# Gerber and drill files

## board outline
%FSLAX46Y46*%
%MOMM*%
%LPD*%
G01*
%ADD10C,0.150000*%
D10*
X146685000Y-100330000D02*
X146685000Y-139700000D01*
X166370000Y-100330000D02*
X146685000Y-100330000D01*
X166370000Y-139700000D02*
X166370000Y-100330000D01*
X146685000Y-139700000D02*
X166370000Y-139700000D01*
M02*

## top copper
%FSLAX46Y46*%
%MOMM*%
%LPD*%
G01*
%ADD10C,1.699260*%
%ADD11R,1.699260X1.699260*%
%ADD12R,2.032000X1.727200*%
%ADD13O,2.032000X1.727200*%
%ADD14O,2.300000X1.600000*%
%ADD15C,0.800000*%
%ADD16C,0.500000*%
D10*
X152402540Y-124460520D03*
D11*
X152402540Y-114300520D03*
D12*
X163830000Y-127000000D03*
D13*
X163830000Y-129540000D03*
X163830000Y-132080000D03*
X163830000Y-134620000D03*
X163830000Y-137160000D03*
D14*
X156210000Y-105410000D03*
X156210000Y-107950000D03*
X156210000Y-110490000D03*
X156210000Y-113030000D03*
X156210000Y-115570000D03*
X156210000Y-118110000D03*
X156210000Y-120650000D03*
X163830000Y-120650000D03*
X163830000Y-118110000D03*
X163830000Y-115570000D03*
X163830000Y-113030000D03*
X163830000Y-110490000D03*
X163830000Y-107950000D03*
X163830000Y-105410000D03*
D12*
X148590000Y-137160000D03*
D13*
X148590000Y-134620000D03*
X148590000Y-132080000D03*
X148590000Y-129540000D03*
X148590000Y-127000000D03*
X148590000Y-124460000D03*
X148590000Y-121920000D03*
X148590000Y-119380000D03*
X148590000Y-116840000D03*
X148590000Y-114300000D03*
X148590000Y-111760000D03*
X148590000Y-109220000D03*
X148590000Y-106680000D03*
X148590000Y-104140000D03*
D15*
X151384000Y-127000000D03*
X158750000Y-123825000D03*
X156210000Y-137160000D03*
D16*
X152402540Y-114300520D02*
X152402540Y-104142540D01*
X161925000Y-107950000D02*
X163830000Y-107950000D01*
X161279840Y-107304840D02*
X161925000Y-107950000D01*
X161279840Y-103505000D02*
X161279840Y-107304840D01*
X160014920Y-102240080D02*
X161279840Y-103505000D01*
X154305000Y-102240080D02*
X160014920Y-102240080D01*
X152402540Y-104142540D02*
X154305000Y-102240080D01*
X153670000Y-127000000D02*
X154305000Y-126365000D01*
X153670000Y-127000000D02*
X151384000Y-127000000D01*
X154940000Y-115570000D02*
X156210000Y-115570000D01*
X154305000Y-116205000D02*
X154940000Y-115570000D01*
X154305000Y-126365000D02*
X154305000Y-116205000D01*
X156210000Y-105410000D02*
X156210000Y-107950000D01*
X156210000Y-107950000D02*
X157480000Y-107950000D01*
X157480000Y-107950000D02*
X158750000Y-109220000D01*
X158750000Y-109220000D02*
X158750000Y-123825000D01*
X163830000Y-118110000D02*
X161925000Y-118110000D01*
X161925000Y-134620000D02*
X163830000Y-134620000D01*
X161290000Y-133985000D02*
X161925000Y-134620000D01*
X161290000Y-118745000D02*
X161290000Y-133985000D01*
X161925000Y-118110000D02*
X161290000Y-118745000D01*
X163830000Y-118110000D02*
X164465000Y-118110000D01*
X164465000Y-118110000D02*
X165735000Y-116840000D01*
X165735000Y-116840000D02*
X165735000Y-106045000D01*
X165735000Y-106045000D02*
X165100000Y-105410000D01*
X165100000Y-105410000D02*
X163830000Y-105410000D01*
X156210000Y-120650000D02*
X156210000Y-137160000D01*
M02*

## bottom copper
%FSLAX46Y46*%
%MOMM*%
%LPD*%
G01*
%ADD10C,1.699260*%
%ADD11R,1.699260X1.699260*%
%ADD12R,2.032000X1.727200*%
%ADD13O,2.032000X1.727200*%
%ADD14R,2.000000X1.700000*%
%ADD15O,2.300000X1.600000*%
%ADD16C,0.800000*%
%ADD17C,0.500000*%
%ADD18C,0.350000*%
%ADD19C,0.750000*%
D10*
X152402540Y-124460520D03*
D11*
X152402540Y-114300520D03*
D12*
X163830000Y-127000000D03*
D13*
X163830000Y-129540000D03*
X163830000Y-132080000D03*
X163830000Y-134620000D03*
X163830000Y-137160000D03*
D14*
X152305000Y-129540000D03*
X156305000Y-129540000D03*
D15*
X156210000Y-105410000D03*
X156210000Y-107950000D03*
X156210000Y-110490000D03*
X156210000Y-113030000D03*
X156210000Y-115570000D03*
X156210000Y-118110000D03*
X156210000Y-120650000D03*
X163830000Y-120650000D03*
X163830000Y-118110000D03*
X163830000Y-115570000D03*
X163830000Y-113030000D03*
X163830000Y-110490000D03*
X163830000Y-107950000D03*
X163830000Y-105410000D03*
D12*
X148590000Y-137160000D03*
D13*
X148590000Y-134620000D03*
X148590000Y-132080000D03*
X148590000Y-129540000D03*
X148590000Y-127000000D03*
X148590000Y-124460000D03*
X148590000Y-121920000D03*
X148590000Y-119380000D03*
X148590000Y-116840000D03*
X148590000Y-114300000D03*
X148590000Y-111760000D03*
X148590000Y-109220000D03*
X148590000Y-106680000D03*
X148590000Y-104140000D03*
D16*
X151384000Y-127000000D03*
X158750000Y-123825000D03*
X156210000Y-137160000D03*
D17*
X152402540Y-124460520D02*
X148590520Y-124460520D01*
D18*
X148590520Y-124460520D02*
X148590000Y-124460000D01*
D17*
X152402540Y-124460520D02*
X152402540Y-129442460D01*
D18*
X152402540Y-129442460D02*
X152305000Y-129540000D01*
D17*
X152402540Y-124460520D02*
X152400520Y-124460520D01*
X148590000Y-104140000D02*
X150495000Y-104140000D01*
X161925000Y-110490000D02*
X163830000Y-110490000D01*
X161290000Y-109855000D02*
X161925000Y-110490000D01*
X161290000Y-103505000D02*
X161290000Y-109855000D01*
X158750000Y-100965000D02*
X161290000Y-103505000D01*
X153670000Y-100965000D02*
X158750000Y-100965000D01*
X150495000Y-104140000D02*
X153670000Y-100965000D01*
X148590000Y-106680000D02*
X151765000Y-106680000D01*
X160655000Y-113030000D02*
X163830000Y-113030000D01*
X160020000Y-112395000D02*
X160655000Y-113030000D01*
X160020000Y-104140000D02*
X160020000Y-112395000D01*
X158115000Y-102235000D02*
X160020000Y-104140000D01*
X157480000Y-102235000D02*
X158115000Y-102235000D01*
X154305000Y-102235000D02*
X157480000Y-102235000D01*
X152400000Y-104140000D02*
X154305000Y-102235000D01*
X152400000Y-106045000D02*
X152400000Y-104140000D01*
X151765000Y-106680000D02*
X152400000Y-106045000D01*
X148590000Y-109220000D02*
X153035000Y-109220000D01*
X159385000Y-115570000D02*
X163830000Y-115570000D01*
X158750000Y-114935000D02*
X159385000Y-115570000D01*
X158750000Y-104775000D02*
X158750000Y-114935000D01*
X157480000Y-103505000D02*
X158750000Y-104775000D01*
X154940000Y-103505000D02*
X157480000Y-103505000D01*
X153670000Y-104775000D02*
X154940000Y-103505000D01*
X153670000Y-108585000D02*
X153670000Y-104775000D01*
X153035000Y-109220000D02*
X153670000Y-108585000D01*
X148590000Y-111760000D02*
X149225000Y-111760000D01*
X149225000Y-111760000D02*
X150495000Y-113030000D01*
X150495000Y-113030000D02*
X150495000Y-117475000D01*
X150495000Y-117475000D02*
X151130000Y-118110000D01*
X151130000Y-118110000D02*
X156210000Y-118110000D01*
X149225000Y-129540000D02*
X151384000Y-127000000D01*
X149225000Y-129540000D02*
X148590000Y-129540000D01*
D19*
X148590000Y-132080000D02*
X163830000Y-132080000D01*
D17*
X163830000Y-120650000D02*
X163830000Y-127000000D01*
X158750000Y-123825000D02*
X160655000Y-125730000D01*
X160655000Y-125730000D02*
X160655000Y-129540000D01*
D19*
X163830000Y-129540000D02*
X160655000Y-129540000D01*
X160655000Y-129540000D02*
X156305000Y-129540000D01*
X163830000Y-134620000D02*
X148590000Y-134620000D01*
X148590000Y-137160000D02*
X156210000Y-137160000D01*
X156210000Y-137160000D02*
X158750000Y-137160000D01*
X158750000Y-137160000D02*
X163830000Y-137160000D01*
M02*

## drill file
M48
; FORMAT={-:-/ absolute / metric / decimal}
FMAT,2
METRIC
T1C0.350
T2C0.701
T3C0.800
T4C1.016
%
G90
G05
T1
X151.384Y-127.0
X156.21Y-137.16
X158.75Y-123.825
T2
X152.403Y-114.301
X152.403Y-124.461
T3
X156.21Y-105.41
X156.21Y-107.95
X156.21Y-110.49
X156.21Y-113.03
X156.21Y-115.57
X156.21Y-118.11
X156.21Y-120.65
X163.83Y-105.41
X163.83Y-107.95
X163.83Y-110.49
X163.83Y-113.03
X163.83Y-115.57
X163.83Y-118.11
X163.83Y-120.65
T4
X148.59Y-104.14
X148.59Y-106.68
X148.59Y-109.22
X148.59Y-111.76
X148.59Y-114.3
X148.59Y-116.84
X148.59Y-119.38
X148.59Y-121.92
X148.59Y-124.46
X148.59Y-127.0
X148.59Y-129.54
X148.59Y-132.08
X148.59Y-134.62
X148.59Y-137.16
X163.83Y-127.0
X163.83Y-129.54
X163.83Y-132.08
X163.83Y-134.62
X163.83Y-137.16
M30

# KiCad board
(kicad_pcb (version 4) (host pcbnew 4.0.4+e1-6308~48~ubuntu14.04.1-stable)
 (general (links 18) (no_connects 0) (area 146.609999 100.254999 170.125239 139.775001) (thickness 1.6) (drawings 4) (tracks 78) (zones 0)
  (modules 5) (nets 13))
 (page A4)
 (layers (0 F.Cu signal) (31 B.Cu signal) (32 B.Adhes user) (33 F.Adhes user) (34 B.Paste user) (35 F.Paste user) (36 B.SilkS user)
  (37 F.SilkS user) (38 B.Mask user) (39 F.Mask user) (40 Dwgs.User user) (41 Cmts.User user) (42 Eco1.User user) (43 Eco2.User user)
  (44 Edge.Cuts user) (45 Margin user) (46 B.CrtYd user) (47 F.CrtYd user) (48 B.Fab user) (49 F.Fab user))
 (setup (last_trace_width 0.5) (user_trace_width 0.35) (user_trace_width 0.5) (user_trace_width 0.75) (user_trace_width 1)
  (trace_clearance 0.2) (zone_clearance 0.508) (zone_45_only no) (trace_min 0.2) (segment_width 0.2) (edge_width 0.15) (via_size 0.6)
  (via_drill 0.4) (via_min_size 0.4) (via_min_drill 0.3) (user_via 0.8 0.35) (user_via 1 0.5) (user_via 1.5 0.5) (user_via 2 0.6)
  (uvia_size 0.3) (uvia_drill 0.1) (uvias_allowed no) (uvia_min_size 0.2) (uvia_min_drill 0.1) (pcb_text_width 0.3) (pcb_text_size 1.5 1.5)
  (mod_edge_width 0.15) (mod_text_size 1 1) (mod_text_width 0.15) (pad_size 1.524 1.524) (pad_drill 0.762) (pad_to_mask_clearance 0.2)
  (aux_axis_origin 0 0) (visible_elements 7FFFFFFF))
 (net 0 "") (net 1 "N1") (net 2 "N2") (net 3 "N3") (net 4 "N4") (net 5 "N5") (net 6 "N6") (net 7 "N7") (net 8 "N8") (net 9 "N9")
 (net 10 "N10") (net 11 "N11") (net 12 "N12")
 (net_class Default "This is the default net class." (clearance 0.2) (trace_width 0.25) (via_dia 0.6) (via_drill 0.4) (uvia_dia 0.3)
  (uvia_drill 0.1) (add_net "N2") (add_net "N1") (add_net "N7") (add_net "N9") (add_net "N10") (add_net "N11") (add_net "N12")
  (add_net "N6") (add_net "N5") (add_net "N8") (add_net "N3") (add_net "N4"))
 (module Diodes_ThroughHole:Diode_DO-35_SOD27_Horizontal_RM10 (layer F.Cu) (at 152.4 114.3 270)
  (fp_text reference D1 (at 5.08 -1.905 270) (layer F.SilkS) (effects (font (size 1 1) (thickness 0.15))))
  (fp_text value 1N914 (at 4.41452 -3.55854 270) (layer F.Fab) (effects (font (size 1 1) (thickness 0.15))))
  (pad 2 thru_hole circle (at 10.16052 -0.00254 90) (size 1.69926 1.69926) (drill 0.70104) (layers *.Cu *.Mask F.SilkS) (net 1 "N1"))
  (pad 1 thru_hole rect (at 0.00052 -0.00254 90) (size 1.69926 1.69926) (drill 0.70104) (layers *.Cu *.Mask F.SilkS) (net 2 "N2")))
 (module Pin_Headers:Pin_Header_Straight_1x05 (layer B.Cu) (at 163.83 127 180)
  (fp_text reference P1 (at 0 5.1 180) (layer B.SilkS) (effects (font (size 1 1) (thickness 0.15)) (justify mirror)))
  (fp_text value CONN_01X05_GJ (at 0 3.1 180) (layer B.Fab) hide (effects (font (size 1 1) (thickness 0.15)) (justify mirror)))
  (pad 1 thru_hole rect (at 0 0 180) (size 2.032 1.7272) (drill 1.016) (layers *.Cu *.Mask B.SilkS) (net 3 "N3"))
  (pad 2 thru_hole oval (at 0 -2.54 180) (size 2.032 1.7272) (drill 1.016) (layers *.Cu *.Mask B.SilkS) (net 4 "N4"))
  (pad 3 thru_hole oval (at 0 -5.08 180) (size 2.032 1.7272) (drill 1.016) (layers *.Cu *.Mask B.SilkS) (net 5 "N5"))
  (pad 4 thru_hole oval (at 0 -7.62 180) (size 2.032 1.7272) (drill 1.016) (layers *.Cu *.Mask B.SilkS) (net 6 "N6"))
  (pad 5 thru_hole oval (at 0 -10.16 180) (size 2.032 1.7272) (drill 1.016) (layers *.Cu *.Mask B.SilkS) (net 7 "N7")))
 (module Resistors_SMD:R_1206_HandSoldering (layer B.Cu) (at 154.305 129.54)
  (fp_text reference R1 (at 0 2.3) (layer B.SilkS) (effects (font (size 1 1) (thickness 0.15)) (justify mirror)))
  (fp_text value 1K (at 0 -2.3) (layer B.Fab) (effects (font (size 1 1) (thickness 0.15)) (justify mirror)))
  (pad 1 smd rect (at -2 0) (size 2 1.7) (layers B.Cu B.Paste B.Mask) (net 1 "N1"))
  (pad 2 smd rect (at 2 0) (size 2 1.7) (layers B.Cu B.Paste B.Mask) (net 4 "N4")))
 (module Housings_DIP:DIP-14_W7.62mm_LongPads (layer F.Cu) (at 156.21 105.41)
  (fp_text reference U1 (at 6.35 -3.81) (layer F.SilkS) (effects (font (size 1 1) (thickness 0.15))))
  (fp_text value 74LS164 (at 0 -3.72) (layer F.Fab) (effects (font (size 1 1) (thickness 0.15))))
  (pad 1 thru_hole oval (at 0 0) (size 2.3 1.6) (drill 0.8) (layers *.Cu *.Mask F.SilkS) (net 4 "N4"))
  (pad 2 thru_hole oval (at 0 2.54) (size 2.3 1.6) (drill 0.8) (layers *.Cu *.Mask F.SilkS) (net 4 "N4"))
  (pad 3 thru_hole oval (at 0 5.08) (size 2.3 1.6) (drill 0.8) (layers *.Cu *.Mask F.SilkS))
  (pad 4 thru_hole oval (at 0 7.62) (size 2.3 1.6) (drill 0.8) (layers *.Cu *.Mask F.SilkS))
  (pad 5 thru_hole oval (at 0 10.16) (size 2.3 1.6) (drill 0.8) (layers *.Cu *.Mask F.SilkS) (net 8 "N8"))
  (pad 6 thru_hole oval (at 0 12.7) (size 2.3 1.6) (drill 0.8) (layers *.Cu *.Mask F.SilkS) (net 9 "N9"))
  (pad 7 thru_hole oval (at 0 15.24) (size 2.3 1.6) (drill 0.8) (layers *.Cu *.Mask F.SilkS) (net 7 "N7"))
  (pad 8 thru_hole oval (at 7.62 15.24) (size 2.3 1.6) (drill 0.8) (layers *.Cu *.Mask F.SilkS) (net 3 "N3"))
  (pad 9 thru_hole oval (at 7.62 12.7) (size 2.3 1.6) (drill 0.8) (layers *.Cu *.Mask F.SilkS) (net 6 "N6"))
  (pad 10 thru_hole oval (at 7.62 10.16) (size 2.3 1.6) (drill 0.8) (layers *.Cu *.Mask F.SilkS) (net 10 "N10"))
  (pad 11 thru_hole oval (at 7.62 7.62) (size 2.3 1.6) (drill 0.8) (layers *.Cu *.Mask F.SilkS) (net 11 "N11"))
  (pad 12 thru_hole oval (at 7.62 5.08) (size 2.3 1.6) (drill 0.8) (layers *.Cu *.Mask F.SilkS) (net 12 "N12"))
  (pad 13 thru_hole oval (at 7.62 2.54) (size 2.3 1.6) (drill 0.8) (layers *.Cu *.Mask F.SilkS) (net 2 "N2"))
  (pad 14 thru_hole oval (at 7.62 0) (size 2.3 1.6) (drill 0.8) (layers *.Cu *.Mask F.SilkS) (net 6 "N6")))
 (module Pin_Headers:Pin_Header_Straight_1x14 (layer F.Cu) (at 148.59 137.16 180)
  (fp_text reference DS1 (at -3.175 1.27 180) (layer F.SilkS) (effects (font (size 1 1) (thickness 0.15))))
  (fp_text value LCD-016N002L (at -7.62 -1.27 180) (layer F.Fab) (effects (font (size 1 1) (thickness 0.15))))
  (pad 1 thru_hole rect (at 0 0 180) (size 2.032 1.7272) (drill 1.016) (layers *.Cu *.Mask F.SilkS) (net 7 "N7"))
  (pad 2 thru_hole oval (at 0 2.54 180) (size 2.032 1.7272) (drill 1.016) (layers *.Cu *.Mask F.SilkS) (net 6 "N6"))
  (pad 3 thru_hole oval (at 0 5.08 180) (size 2.032 1.7272) (drill 1.016) (layers *.Cu *.Mask F.SilkS) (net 5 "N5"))
  (pad 4 thru_hole oval (at 0 7.62 180) (size 2.032 1.7272) (drill 1.016) (layers *.Cu *.Mask F.SilkS) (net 8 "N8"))
  (pad 5 thru_hole oval (at 0 10.16 180) (size 2.032 1.7272) (drill 1.016) (layers *.Cu *.Mask F.SilkS))
  (pad 6 thru_hole oval (at 0 12.7 180) (size 2.032 1.7272) (drill 1.016) (layers *.Cu *.Mask F.SilkS) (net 1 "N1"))
  (pad 7 thru_hole oval (at 0 15.24 180) (size 2.032 1.7272) (drill 1.016) (layers *.Cu *.Mask F.SilkS))
  (pad 8 thru_hole oval (at 0 17.78 180) (size 2.032 1.7272) (drill 1.016) (layers *.Cu *.Mask F.SilkS))
  (pad 9 thru_hole oval (at 0 20.32 180) (size 2.032 1.7272) (drill 1.016) (layers *.Cu *.Mask F.SilkS))
  (pad 10 thru_hole oval (at 0 22.86 180) (size 2.032 1.7272) (drill 1.016) (layers *.Cu *.Mask F.SilkS))
  (pad 11 thru_hole oval (at 0 25.4 180) (size 2.032 1.7272) (drill 1.016) (layers *.Cu *.Mask F.SilkS) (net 9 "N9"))
  (pad 12 thru_hole oval (at 0 27.94 180) (size 2.032 1.7272) (drill 1.016) (layers *.Cu *.Mask F.SilkS) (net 10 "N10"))
  (pad 13 thru_hole oval (at 0 30.48 180) (size 2.032 1.7272) (drill 1.016) (layers *.Cu *.Mask F.SilkS) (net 11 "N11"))
  (pad 14 thru_hole oval (at 0 33.02 180) (size 2.032 1.7272) (drill 1.016) (layers *.Cu *.Mask F.SilkS) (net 12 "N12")))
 (gr_line (start 146.685 100.33) (end 146.685 139.7) (angle 90) (layer Edge.Cuts) (width 0.15))
 (gr_line (start 166.37 100.33) (end 146.685 100.33) (angle 90) (layer Edge.Cuts) (width 0.15))
 (gr_line (start 166.37 139.7) (end 166.37 100.33) (angle 90) (layer Edge.Cuts) (width 0.15))
 (gr_line (start 146.685 139.7) (end 166.37 139.7) (angle 90) (layer Edge.Cuts) (width 0.15))
 (segment (start 152.40254 124.46052) (end 148.59052 124.46052) (width 0.5) (layer B.Cu) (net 1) (status 10))
 (segment (start 148.59052 124.46052) (end 148.59 124.46) (width 0.35) (layer B.Cu) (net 1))
 (segment (start 152.40254 124.46052) (end 152.40254 129.44246) (width 0.5) (layer B.Cu) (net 1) (status 20))
 (segment (start 152.40254 129.44246) (end 152.305 129.54) (width 0.35) (layer B.Cu) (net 1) (status 30))
 (segment (start 152.40254 124.46052) (end 152.40052 124.46052) (width 0.5) (layer B.Cu) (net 1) (status 30))
 (segment (start 152.40254 114.30052) (end 152.40254 104.14254) (width 0.5) (layer F.Cu) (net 2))
 (segment (start 161.925 107.95) (end 163.83 107.95) (width 0.5) (layer F.Cu) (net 2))
 (segment (start 161.27984 107.30484) (end 161.925 107.95) (width 0.5) (layer F.Cu) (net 2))
 (segment (start 161.27984 103.505) (end 161.27984 107.30484) (width 0.5) (layer F.Cu) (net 2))
 (segment (start 160.01492 102.24008) (end 161.27984 103.505) (width 0.5) (layer F.Cu) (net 2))
 (segment (start 154.305 102.24008) (end 160.01492 102.24008) (width 0.5) (layer F.Cu) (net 2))
 (segment (start 152.40254 104.14254) (end 154.305 102.24008) (width 0.5) (layer F.Cu) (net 2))
 (segment (start 148.59 104.14) (end 150.495 104.14) (width 0.5) (layer B.Cu) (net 12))
 (segment (start 161.925 110.49) (end 163.83 110.49) (width 0.5) (layer B.Cu) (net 12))
 (segment (start 161.29 109.855) (end 161.925 110.49) (width 0.5) (layer B.Cu) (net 12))
 (segment (start 161.29 103.505) (end 161.29 109.855) (width 0.5) (layer B.Cu) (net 12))
 (segment (start 158.75 100.965) (end 161.29 103.505) (width 0.5) (layer B.Cu) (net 12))
 (segment (start 153.67 100.965) (end 158.75 100.965) (width 0.5) (layer B.Cu) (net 12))
 (segment (start 150.495 104.14) (end 153.67 100.965) (width 0.5) (layer B.Cu) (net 12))
 (segment (start 148.59 106.68) (end 151.765 106.68) (width 0.5) (layer B.Cu) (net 11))
 (segment (start 160.655 113.03) (end 163.83 113.03) (width 0.5) (layer B.Cu) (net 11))
 (segment (start 160.02 112.395) (end 160.655 113.03) (width 0.5) (layer B.Cu) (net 11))
 (segment (start 160.02 104.14) (end 160.02 112.395) (width 0.5) (layer B.Cu) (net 11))
 (segment (start 158.115 102.235) (end 160.02 104.14) (width 0.5) (layer B.Cu) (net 11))
 (segment (start 157.48 102.235) (end 158.115 102.235) (width 0.5) (layer B.Cu) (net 11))
 (segment (start 154.305 102.235) (end 157.48 102.235) (width 0.5) (layer B.Cu) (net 11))
 (segment (start 152.4 104.14) (end 154.305 102.235) (width 0.5) (layer B.Cu) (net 11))
 (segment (start 152.4 106.045) (end 152.4 104.14) (width 0.5) (layer B.Cu) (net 11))
 (segment (start 151.765 106.68) (end 152.4 106.045) (width 0.5) (layer B.Cu) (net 11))
 (segment (start 148.59 109.22) (end 153.035 109.22) (width 0.5) (layer B.Cu) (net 10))
 (segment (start 159.385 115.57) (end 163.83 115.57) (width 0.5) (layer B.Cu) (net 10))
 (segment (start 158.75 114.935) (end 159.385 115.57) (width 0.5) (layer B.Cu) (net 10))
 (segment (start 158.75 104.775) (end 158.75 114.935) (width 0.5) (layer B.Cu) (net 10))
 (segment (start 157.48 103.505) (end 158.75 104.775) (width 0.5) (layer B.Cu) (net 10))
 (segment (start 154.94 103.505) (end 157.48 103.505) (width 0.5) (layer B.Cu) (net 10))
 (segment (start 153.67 104.775) (end 154.94 103.505) (width 0.5) (layer B.Cu) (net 10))
 (segment (start 153.67 108.585) (end 153.67 104.775) (width 0.5) (layer B.Cu) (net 10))
 (segment (start 153.035 109.22) (end 153.67 108.585) (width 0.5) (layer B.Cu) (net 10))
 (segment (start 148.59 111.76) (end 149.225 111.76) (width 0.5) (layer B.Cu) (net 9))
 (segment (start 149.225 111.76) (end 150.495 113.03) (width 0.5) (layer B.Cu) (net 9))
 (segment (start 150.495 113.03) (end 150.495 117.475) (width 0.5) (layer B.Cu) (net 9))
 (segment (start 150.495 117.475) (end 151.13 118.11) (width 0.5) (layer B.Cu) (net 9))
 (segment (start 151.13 118.11) (end 156.21 118.11) (width 0.5) (layer B.Cu) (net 9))
 (segment (start 153.67 127) (end 154.305 126.365) (width 0.5) (layer F.Cu) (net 8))
 (segment (start 153.67 127) (end 151.384 127) (width 0.5) (layer F.Cu) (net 8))
 (via (at 151.384 127) (size 0.8) (drill 0.35) (layers F.Cu B.Cu) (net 8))
 (segment (start 149.225 129.54) (end 151.384 127) (width 0.5) (layer B.Cu) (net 8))
 (segment (start 154.94 115.57) (end 156.21 115.57) (width 0.5) (layer F.Cu) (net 8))
 (segment (start 154.305 116.205) (end 154.94 115.57) (width 0.5) (layer F.Cu) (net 8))
 (segment (start 154.305 126.365) (end 154.305 116.205) (width 0.5) (layer F.Cu) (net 8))
 (segment (start 149.225 129.54) (end 148.59 129.54) (width 0.5) (layer B.Cu) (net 8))
 (segment (start 148.59 132.08) (end 163.83 132.08) (width 0.75) (layer B.Cu) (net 5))
 (segment (start 163.83 120.65) (end 163.83 127) (width 0.5) (layer B.Cu) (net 3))
 (segment (start 156.21 105.41) (end 156.21 107.95) (width 0.5) (layer F.Cu) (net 4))
 (segment (start 156.21 107.95) (end 157.48 107.95) (width 0.5) (layer F.Cu) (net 4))
 (segment (start 157.48 107.95) (end 158.75 109.22) (width 0.5) (layer F.Cu) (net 4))
 (segment (start 158.75 109.22) (end 158.75 123.825) (width 0.5) (layer F.Cu) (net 4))
 (via (at 158.75 123.825) (size 0.8) (drill 0.35) (layers F.Cu B.Cu) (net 4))
 (segment (start 158.75 123.825) (end 160.655 125.73) (width 0.5) (layer B.Cu) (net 4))
 (segment (start 160.655 125.73) (end 160.655 129.54) (width 0.5) (layer B.Cu) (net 4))
 (segment (start 163.83 129.54) (end 160.655 129.54) (width 0.75) (layer B.Cu) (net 4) (status 20))
 (segment (start 160.655 129.54) (end 156.305 129.54) (width 0.75) (layer B.Cu) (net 4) (status 20))
 (segment (start 163.83 118.11) (end 161.925 118.11) (width 0.5) (layer F.Cu) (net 6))
 (segment (start 161.925 134.62) (end 163.83 134.62) (width 0.5) (layer F.Cu) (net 6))
 (segment (start 161.29 133.985) (end 161.925 134.62) (width 0.5) (layer F.Cu) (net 6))
 (segment (start 161.29 118.745) (end 161.29 133.985) (width 0.5) (layer F.Cu) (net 6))
 (segment (start 161.925 118.11) (end 161.29 118.745) (width 0.5) (layer F.Cu) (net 6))
 (segment (start 163.83 118.11) (end 164.465 118.11) (width 0.5) (layer F.Cu) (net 6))
 (segment (start 164.465 118.11) (end 165.735 116.84) (width 0.5) (layer F.Cu) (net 6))
 (segment (start 165.735 116.84) (end 165.735 106.045) (width 0.5) (layer F.Cu) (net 6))
 (segment (start 165.735 106.045) (end 165.1 105.41) (width 0.5) (layer F.Cu) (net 6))
 (segment (start 165.1 105.41) (end 163.83 105.41) (width 0.5) (layer F.Cu) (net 6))
 (segment (start 163.83 134.62) (end 148.59 134.62) (width 0.75) (layer B.Cu) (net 6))
 (segment (start 156.21 120.65) (end 156.21 137.16) (width 0.5) (layer F.Cu) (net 7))
 (via (at 156.21 137.16) (size 0.8) (drill 0.35) (layers F.Cu B.Cu) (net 7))
 (segment (start 148.59 137.16) (end 156.21 137.16) (width 0.75) (layer B.Cu) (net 7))
 (segment (start 156.21 137.16) (end 158.75 137.16) (width 0.75) (layer B.Cu) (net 7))
 (segment (start 158.75 137.16) (end 163.83 137.16) (width 0.75) (layer B.Cu) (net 7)))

